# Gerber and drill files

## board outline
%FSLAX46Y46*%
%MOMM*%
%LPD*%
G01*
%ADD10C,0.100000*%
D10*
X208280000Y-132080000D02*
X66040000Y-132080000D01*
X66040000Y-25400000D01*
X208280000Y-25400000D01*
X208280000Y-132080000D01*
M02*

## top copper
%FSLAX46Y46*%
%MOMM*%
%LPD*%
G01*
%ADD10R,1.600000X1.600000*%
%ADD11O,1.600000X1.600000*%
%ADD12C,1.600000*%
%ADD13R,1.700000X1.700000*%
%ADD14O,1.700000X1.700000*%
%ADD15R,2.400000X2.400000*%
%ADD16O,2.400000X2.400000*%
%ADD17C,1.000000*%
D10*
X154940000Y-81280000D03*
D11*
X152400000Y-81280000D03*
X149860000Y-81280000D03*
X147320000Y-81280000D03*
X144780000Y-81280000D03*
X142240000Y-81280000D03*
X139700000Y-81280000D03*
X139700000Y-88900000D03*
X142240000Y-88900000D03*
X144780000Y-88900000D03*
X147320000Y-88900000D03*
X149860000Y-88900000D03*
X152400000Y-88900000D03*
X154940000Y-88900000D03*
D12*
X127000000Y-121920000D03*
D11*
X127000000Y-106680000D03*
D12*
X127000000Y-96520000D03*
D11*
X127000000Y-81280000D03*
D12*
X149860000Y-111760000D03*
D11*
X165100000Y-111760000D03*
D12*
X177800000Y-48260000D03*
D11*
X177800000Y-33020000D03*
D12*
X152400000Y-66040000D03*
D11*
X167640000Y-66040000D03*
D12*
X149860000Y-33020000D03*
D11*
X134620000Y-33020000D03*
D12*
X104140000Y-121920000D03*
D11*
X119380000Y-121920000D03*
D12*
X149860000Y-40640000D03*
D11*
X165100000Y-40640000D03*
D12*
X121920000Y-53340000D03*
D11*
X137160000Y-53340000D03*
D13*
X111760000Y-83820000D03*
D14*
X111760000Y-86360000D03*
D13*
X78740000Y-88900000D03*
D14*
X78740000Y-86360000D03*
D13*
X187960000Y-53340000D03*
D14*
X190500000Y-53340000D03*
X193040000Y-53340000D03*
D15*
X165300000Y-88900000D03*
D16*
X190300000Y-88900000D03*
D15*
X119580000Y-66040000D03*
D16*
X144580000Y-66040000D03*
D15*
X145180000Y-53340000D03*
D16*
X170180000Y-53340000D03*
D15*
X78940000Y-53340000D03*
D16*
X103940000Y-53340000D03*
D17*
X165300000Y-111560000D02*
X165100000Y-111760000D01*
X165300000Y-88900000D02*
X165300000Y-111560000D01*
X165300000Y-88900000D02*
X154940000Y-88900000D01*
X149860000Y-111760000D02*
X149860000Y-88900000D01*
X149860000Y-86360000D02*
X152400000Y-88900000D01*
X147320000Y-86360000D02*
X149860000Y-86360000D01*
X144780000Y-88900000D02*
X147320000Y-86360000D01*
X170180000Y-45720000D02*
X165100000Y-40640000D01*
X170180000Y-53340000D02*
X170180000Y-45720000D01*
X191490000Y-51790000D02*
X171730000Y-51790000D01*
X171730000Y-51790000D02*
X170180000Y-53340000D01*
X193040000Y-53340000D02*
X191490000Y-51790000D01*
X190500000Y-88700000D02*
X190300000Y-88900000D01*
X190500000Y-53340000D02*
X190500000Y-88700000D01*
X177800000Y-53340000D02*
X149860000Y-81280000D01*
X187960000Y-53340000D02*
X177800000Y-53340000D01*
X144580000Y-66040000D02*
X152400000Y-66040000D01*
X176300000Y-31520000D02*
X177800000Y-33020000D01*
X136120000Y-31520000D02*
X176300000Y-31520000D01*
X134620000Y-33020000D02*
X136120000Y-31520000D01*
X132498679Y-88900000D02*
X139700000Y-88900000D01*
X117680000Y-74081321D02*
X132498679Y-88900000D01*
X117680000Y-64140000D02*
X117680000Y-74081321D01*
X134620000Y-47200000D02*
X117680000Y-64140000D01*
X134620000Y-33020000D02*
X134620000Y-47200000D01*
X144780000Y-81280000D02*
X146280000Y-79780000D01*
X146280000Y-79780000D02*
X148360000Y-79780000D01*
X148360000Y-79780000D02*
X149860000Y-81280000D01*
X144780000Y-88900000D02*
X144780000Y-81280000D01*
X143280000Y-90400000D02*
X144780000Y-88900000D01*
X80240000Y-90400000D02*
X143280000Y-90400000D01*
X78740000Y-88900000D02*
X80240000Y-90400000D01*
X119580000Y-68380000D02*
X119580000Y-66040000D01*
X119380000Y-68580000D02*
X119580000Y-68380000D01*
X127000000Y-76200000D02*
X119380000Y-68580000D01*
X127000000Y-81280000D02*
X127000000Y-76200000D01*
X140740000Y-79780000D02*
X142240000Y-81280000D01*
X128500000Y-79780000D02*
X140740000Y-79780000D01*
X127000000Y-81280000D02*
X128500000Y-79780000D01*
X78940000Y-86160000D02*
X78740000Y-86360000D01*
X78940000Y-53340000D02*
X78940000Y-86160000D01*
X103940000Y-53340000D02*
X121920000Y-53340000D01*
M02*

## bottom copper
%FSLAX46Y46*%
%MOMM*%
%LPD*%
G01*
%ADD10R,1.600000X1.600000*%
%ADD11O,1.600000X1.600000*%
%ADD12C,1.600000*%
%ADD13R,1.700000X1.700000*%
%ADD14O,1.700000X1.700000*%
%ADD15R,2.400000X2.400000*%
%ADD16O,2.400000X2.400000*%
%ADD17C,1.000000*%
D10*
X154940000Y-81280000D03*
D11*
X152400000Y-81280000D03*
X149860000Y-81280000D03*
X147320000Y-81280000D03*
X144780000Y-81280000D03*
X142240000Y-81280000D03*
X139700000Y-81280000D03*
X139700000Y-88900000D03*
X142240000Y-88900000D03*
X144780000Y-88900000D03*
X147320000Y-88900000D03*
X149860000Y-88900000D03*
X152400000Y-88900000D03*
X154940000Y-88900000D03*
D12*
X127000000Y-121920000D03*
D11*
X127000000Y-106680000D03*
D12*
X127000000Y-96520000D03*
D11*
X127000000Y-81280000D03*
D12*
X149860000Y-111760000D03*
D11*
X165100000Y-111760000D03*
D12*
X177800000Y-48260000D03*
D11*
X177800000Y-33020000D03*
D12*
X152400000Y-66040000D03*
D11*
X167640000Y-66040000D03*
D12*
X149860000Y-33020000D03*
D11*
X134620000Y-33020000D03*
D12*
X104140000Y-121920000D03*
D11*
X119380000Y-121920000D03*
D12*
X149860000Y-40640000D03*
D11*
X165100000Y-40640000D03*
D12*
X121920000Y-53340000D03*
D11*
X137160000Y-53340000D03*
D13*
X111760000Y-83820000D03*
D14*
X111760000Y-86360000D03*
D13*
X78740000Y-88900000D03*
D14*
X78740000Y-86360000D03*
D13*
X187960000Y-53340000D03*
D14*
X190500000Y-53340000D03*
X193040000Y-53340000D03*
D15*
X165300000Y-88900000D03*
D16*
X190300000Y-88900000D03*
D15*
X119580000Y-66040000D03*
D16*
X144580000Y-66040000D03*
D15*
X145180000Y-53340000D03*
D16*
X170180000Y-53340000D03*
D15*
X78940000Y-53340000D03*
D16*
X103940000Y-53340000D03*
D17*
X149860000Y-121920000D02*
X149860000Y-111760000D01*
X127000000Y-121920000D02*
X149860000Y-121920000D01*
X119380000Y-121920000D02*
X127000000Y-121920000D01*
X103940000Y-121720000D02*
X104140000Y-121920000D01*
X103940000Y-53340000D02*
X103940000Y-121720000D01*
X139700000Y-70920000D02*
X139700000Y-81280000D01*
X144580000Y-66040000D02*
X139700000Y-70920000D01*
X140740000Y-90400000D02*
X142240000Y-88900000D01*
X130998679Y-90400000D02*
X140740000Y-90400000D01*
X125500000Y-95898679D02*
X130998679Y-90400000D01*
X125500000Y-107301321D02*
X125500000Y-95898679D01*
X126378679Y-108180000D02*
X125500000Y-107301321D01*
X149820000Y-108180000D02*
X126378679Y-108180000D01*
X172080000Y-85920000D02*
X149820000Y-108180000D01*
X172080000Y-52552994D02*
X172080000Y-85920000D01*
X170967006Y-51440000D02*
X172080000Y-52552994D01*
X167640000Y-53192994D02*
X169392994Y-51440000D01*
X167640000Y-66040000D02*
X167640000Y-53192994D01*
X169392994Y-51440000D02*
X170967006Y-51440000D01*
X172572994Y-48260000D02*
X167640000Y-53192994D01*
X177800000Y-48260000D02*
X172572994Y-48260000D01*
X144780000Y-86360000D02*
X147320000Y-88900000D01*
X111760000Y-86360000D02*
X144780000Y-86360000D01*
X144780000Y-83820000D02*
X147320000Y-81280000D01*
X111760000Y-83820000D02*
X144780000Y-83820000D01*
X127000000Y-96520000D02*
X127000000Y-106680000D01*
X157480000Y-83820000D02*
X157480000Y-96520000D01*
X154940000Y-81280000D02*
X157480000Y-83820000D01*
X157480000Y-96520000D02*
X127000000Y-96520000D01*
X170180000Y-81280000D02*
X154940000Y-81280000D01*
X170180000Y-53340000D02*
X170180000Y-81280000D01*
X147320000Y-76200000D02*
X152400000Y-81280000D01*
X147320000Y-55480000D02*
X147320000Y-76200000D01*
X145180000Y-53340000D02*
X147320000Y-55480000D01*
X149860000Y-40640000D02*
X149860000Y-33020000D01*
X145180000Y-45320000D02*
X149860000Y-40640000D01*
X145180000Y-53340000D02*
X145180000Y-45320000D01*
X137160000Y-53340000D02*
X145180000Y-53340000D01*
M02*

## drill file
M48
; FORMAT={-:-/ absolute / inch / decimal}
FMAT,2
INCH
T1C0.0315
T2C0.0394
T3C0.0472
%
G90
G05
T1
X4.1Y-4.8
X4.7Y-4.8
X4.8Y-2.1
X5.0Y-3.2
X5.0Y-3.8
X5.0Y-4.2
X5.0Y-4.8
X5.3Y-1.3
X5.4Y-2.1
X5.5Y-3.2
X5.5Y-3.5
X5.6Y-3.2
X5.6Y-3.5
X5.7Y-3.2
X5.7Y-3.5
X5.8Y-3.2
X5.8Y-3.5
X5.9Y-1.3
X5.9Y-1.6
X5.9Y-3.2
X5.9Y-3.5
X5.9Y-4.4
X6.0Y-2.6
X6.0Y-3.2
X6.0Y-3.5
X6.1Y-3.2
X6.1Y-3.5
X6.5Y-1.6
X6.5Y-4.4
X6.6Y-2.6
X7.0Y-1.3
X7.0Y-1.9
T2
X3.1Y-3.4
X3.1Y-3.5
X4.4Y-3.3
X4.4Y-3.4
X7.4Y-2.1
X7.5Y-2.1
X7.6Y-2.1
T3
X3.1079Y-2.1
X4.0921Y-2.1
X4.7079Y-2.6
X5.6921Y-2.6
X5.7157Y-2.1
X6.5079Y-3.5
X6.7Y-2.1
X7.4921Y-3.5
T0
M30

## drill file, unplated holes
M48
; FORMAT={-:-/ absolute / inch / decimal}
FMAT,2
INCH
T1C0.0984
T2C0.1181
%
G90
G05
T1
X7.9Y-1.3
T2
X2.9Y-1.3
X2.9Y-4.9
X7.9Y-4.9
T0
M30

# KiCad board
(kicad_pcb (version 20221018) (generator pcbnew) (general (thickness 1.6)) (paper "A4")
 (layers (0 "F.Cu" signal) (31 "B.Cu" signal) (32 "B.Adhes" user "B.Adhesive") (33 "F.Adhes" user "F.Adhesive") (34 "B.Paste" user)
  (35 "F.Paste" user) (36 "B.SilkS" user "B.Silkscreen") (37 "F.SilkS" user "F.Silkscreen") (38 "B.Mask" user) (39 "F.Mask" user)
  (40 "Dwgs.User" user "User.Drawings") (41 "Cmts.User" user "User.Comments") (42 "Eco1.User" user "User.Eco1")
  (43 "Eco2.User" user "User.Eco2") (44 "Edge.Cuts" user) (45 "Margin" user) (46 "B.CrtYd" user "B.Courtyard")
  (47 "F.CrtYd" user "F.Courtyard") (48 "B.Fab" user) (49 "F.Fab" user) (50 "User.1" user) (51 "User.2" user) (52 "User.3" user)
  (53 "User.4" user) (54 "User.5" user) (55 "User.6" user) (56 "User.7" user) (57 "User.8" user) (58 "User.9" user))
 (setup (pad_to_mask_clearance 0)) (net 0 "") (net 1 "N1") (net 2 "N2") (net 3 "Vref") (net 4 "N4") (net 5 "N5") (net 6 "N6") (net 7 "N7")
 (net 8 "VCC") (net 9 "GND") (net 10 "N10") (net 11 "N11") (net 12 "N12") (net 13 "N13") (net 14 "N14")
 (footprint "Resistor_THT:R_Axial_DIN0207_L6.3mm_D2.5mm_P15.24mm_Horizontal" (layer "F.Cu") (at 152.4 66.04)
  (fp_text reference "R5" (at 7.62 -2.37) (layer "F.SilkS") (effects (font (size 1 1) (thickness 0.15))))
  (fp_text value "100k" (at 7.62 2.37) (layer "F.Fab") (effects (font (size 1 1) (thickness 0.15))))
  (pad "1" thru_hole circle (at 0 0) (size 1.6 1.6) (drill 0.8) (layers "*.Cu" "*.Mask") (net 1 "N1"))
  (pad "2" thru_hole oval (at 15.24 0) (size 1.6 1.6) (drill 0.8) (layers "*.Cu" "*.Mask") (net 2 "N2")))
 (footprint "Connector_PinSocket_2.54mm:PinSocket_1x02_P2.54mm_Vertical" (layer "F.Cu") (at 78.74 88.9 180)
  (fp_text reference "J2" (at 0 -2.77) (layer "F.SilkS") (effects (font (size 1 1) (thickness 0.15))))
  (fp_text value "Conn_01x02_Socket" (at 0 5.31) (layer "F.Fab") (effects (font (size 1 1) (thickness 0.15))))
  (pad "1" thru_hole rect (at 0 0 180) (size 1.7 1.7) (drill 1) (layers "*.Cu" "*.Mask") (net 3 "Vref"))
  (pad "2" thru_hole oval (at 0 2.54 180) (size 1.7 1.7) (drill 1) (layers "*.Cu" "*.Mask") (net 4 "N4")))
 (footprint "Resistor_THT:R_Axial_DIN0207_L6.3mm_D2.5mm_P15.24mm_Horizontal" (layer "F.Cu") (at 121.92 53.34)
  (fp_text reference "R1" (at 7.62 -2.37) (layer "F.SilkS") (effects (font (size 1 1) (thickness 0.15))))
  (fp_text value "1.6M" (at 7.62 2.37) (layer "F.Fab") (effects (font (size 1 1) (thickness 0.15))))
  (pad "1" thru_hole circle (at 0 0) (size 1.6 1.6) (drill 0.8) (layers "*.Cu" "*.Mask") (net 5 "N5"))
  (pad "2" thru_hole oval (at 15.24 0) (size 1.6 1.6) (drill 0.8) (layers "*.Cu" "*.Mask") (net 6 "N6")))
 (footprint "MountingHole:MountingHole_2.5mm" (layer "F.Cu") (at 200.66 33.02)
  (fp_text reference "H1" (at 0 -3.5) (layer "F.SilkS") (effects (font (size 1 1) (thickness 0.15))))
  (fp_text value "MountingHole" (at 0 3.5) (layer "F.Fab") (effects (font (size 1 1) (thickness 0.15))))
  (pad "" np_thru_hole circle (at 0 0) (size 2.5 2.5) (drill 2.5) (layers "*.Cu" "*.Mask")))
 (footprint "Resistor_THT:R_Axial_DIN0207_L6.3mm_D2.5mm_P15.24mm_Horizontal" (layer "F.Cu") (at 149.86 40.64)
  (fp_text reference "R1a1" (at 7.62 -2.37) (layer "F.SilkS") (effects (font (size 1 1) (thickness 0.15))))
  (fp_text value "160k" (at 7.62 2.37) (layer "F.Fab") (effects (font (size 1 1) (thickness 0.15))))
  (pad "1" thru_hole circle (at 0 0) (size 1.6 1.6) (drill 0.8) (layers "*.Cu" "*.Mask") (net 6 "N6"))
  (pad "2" thru_hole oval (at 15.24 0) (size 1.6 1.6) (drill 0.8) (layers "*.Cu" "*.Mask") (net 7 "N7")))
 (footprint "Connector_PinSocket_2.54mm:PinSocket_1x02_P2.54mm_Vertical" (layer "F.Cu") (at 111.76 83.82)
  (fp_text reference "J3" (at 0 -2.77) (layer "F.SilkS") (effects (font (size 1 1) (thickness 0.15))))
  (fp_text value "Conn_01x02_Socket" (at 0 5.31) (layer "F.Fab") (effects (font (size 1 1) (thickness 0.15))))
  (pad "1" thru_hole rect (at 0 0) (size 1.7 1.7) (drill 1) (layers "*.Cu" "*.Mask") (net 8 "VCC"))
  (pad "2" thru_hole oval (at 0 2.54) (size 1.7 1.7) (drill 1) (layers "*.Cu" "*.Mask") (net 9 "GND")))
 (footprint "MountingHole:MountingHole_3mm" (layer "F.Cu") (at 200.66 124.46)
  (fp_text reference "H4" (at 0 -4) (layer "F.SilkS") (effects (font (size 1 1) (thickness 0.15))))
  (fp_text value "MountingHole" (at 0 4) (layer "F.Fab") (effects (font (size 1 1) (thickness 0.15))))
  (pad "" np_thru_hole circle (at 0 0) (size 3 3) (drill 3) (layers "*.Cu" "*.Mask")))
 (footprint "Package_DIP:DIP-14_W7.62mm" (layer "F.Cu") (at 154.94 81.28 -90)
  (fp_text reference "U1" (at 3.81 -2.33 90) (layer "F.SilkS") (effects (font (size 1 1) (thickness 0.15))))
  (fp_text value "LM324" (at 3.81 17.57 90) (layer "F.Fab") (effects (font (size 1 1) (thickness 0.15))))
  (pad "1" thru_hole rect (at 0 0 270) (size 1.6 1.6) (drill 0.8) (layers "*.Cu" "*.Mask") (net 7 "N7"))
  (pad "2" thru_hole oval (at 0 2.54 270) (size 1.6 1.6) (drill 0.8) (layers "*.Cu" "*.Mask") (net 6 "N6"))
  (pad "3" thru_hole oval (at 0 5.08 270) (size 1.6 1.6) (drill 0.8) (layers "*.Cu" "*.Mask") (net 3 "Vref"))
  (pad "4" thru_hole oval (at 0 7.62 270) (size 1.6 1.6) (drill 0.8) (layers "*.Cu" "*.Mask") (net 8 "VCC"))
  (pad "5" thru_hole oval (at 0 10.16 270) (size 1.6 1.6) (drill 0.8) (layers "*.Cu" "*.Mask") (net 3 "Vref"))
  (pad "6" thru_hole oval (at 0 12.7 270) (size 1.6 1.6) (drill 0.8) (layers "*.Cu" "*.Mask") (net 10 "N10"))
  (pad "7" thru_hole oval (at 0 15.24 270) (size 1.6 1.6) (drill 0.8) (layers "*.Cu" "*.Mask") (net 1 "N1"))
  (pad "8" thru_hole oval (at 7.62 15.24 270) (size 1.6 1.6) (drill 0.8) (layers "*.Cu" "*.Mask") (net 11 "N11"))
  (pad "9" thru_hole oval (at 7.62 12.7 270) (size 1.6 1.6) (drill 0.8) (layers "*.Cu" "*.Mask") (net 2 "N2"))
  (pad "10" thru_hole oval (at 7.62 10.16 270) (size 1.6 1.6) (drill 0.8) (layers "*.Cu" "*.Mask") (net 3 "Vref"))
  (pad "11" thru_hole oval (at 7.62 7.62 270) (size 1.6 1.6) (drill 0.8) (layers "*.Cu" "*.Mask") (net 9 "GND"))
  (pad "12" thru_hole oval (at 7.62 5.08 270) (size 1.6 1.6) (drill 0.8) (layers "*.Cu" "*.Mask") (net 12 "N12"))
  (pad "13" thru_hole oval (at 7.62 2.54 270) (size 1.6 1.6) (drill 0.8) (layers "*.Cu" "*.Mask") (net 3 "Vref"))
  (pad "14" thru_hole oval (at 7.62 0 270) (size 1.6 1.6) (drill 0.8) (layers "*.Cu" "*.Mask") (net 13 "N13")))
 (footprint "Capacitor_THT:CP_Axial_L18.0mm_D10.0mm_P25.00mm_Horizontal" (layer "F.Cu") (at 165.3 88.9)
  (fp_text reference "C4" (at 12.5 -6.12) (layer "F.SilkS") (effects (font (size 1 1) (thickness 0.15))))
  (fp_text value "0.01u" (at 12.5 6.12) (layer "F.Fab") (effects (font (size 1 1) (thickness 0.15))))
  (pad "1" thru_hole rect (at 0 0) (size 2.4 2.4) (drill 1.2) (layers "*.Cu" "*.Mask") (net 13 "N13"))
  (pad "2" thru_hole oval (at 25 0) (size 2.4 2.4) (drill 1.2) (layers "*.Cu" "*.Mask") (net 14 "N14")))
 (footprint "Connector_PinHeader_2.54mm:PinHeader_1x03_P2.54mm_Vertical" (layer "F.Cu") (at 187.96 53.34 90)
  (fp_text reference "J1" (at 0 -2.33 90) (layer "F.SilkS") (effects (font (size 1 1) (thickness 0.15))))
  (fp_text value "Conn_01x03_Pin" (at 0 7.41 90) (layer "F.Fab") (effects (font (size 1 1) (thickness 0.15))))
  (pad "1" thru_hole rect (at 0 0 90) (size 1.7 1.7) (drill 1) (layers "*.Cu" "*.Mask") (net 3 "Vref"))
  (pad "2" thru_hole oval (at 0 2.54 90) (size 1.7 1.7) (drill 1) (layers "*.Cu" "*.Mask") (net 14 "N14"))
  (pad "3" thru_hole oval (at 0 5.08 90) (size 1.7 1.7) (drill 1) (layers "*.Cu" "*.Mask") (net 7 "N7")))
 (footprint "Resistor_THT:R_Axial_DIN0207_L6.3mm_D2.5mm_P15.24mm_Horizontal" (layer "F.Cu") (at 104.14 121.92)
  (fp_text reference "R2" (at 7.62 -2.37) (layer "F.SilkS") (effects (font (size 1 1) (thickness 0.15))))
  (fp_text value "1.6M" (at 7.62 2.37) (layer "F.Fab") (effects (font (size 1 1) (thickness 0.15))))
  (pad "1" thru_hole circle (at 0 0) (size 1.6 1.6) (drill 0.8) (layers "*.Cu" "*.Mask") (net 5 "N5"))
  (pad "2" thru_hole oval (at 15.24 0) (size 1.6 1.6) (drill 0.8) (layers "*.Cu" "*.Mask") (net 12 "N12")))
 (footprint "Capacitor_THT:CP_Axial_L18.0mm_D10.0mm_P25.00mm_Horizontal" (layer "F.Cu") (at 78.94 53.34)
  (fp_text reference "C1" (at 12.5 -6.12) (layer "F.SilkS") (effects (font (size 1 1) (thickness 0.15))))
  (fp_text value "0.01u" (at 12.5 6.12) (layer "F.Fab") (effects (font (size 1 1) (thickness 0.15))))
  (pad "1" thru_hole rect (at 0 0) (size 2.4 2.4) (drill 1.2) (layers "*.Cu" "*.Mask") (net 4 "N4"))
  (pad "2" thru_hole oval (at 25 0) (size 2.4 2.4) (drill 1.2) (layers "*.Cu" "*.Mask") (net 5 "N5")))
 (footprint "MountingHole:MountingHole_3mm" (layer "F.Cu") (at 73.66 124.46)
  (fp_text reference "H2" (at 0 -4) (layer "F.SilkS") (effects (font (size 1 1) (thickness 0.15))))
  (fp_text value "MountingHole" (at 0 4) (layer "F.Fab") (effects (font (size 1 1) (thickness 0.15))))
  (pad "" np_thru_hole circle (at 0 0) (size 3 3) (drill 3) (layers "*.Cu" "*.Mask")))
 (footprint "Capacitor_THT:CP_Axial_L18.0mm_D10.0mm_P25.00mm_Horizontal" (layer "F.Cu") (at 145.18 53.34)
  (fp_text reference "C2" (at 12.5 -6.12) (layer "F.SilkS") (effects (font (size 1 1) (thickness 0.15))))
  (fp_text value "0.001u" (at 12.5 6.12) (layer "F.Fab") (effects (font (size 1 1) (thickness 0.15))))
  (pad "1" thru_hole rect (at 0 0) (size 2.4 2.4) (drill 1.2) (layers "*.Cu" "*.Mask") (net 6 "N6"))
  (pad "2" thru_hole oval (at 25 0) (size 2.4 2.4) (drill 1.2) (layers "*.Cu" "*.Mask") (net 7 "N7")))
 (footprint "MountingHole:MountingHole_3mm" (layer "F.Cu") (at 73.66 33.02)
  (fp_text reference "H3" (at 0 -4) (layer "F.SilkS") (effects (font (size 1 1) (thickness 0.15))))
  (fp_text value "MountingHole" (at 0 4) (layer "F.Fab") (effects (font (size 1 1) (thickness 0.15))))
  (pad "" np_thru_hole circle (at 0 0) (size 3 3) (drill 3) (layers "*.Cu" "*.Mask")))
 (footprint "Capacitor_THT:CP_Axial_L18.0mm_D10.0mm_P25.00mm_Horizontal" (layer "F.Cu") (at 119.58 66.04)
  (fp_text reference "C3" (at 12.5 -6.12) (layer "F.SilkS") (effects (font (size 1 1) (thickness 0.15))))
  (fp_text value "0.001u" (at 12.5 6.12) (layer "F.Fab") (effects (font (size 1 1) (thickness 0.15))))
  (pad "1" thru_hole rect (at 0 0) (size 2.4 2.4) (drill 1.2) (layers "*.Cu" "*.Mask") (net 10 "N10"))
  (pad "2" thru_hole oval (at 25 0) (size 2.4 2.4) (drill 1.2) (layers "*.Cu" "*.Mask") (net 1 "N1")))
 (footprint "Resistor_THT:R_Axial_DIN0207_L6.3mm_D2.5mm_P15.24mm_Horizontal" (layer "F.Cu") (at 127 96.52 90)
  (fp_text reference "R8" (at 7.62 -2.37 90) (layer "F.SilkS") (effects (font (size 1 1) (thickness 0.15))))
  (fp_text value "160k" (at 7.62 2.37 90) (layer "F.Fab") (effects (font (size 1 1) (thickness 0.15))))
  (pad "1" thru_hole circle (at 0 0 90) (size 1.6 1.6) (drill 0.8) (layers "*.Cu" "*.Mask") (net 7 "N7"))
  (pad "2" thru_hole oval (at 15.24 0 90) (size 1.6 1.6) (drill 0.8) (layers "*.Cu" "*.Mask") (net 10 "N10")))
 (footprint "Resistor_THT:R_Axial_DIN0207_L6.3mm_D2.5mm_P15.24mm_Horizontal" (layer "F.Cu") (at 149.86 33.02 180)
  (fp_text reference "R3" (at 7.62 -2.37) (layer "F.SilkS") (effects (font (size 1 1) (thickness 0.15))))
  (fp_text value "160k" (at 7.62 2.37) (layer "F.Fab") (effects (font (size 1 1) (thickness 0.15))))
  (pad "1" thru_hole circle (at 0 0 180) (size 1.6 1.6) (drill 0.8) (layers "*.Cu" "*.Mask") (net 6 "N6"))
  (pad "2" thru_hole oval (at 15.24 0 180) (size 1.6 1.6) (drill 0.8) (layers "*.Cu" "*.Mask") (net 11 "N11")))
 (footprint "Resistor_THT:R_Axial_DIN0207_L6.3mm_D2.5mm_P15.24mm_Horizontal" (layer "F.Cu") (at 149.86 111.76)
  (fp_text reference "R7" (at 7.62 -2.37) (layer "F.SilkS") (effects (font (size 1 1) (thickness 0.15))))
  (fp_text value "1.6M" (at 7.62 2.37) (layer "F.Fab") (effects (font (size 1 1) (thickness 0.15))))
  (pad "1" thru_hole circle (at 0 0) (size 1.6 1.6) (drill 0.8) (layers "*.Cu" "*.Mask") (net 12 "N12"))
  (pad "2" thru_hole oval (at 15.24 0) (size 1.6 1.6) (drill 0.8) (layers "*.Cu" "*.Mask") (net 13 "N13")))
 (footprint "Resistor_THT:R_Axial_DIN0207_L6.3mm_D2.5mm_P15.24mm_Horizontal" (layer "F.Cu") (at 177.8 48.26 90)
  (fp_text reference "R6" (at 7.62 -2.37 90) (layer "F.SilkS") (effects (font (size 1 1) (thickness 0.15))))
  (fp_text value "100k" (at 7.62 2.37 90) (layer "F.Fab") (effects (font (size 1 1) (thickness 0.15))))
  (pad "1" thru_hole circle (at 0 0 90) (size 1.6 1.6) (drill 0.8) (layers "*.Cu" "*.Mask") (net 2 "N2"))
  (pad "2" thru_hole oval (at 15.24 0 90) (size 1.6 1.6) (drill 0.8) (layers "*.Cu" "*.Mask") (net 11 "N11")))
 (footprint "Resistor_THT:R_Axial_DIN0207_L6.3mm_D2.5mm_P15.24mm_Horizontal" (layer "F.Cu") (at 127 121.92 90)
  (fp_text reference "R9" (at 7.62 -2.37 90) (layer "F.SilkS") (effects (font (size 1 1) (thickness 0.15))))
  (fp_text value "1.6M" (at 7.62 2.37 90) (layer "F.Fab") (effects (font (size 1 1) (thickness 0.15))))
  (pad "1" thru_hole circle (at 0 0 90) (size 1.6 1.6) (drill 0.8) (layers "*.Cu" "*.Mask") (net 12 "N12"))
  (pad "2" thru_hole oval (at 15.24 0 90) (size 1.6 1.6) (drill 0.8) (layers "*.Cu" "*.Mask") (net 7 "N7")))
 (gr_poly
  (pts (xy 66.04 25.4) (xy 208.28 25.4) (xy 208.28 132.08) (xy 66.04 132.08)) (stroke (width 0.1) (type solid)) (fill none)
  (layer "Edge.Cuts"))
 (segment (start 78.94 86.16) (end 78.74 86.36) (width 1) (layer "F.Cu") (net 4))
 (segment (start 78.94 53.34) (end 78.94 86.16) (width 1) (layer "F.Cu") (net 4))
 (segment (start 103.94 53.34) (end 121.92 53.34) (width 1) (layer "F.Cu") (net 5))
 (segment (start 103.94 53.34) (end 103.94 121.72) (width 1) (layer "B.Cu") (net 5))
 (segment (start 103.94 121.72) (end 104.14 121.92) (width 1) (layer "B.Cu") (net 5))
 (segment (start 147.32 55.48) (end 147.32 76.2) (width 1) (layer "B.Cu") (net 6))
 (segment (start 145.18 53.34) (end 147.32 55.48) (width 1) (layer "B.Cu") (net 6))
 (segment (start 149.86 40.64) (end 149.86 33.02) (width 1) (layer "B.Cu") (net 6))
 (segment (start 137.16 53.34) (end 145.18 53.34) (width 1) (layer "B.Cu") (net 6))
 (segment (start 145.18 45.32) (end 149.86 40.64) (width 1) (layer "B.Cu") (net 6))
 (segment (start 147.32 76.2) (end 152.4 81.28) (width 1) (layer "B.Cu") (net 6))
 (segment (start 145.18 53.34) (end 145.18 45.32) (width 1) (layer "B.Cu") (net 6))
 (segment (start 191.49 51.79) (end 171.73 51.79) (width 1) (layer "F.Cu") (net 7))
 (segment (start 170.18 53.34) (end 170.18 45.72) (width 1) (layer "F.Cu") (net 7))
 (segment (start 171.73 51.79) (end 170.18 53.34) (width 1) (layer "F.Cu") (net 7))
 (segment (start 193.04 53.34) (end 191.49 51.79) (width 1) (layer "F.Cu") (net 7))
 (segment (start 170.18 45.72) (end 165.1 40.64) (width 1) (layer "F.Cu") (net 7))
 (segment (start 154.94 81.28) (end 157.48 83.82) (width 1) (layer "B.Cu") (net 7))
 (segment (start 127 96.52) (end 127 106.68) (width 1) (layer "B.Cu") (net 7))
 (segment (start 157.48 96.52) (end 127 96.52) (width 1) (layer "B.Cu") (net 7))
 (segment (start 170.18 53.34) (end 170.18 81.28) (width 1) (layer "B.Cu") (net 7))
 (segment (start 157.48 83.82) (end 157.48 96.52) (width 1) (layer "B.Cu") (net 7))
 (segment (start 170.18 81.28) (end 154.94 81.28) (width 1) (layer "B.Cu") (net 7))
 (segment (start 128.5 79.78) (end 140.74 79.78) (width 1) (layer "F.Cu") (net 10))
 (segment (start 127 81.28) (end 128.5 79.78) (width 1) (layer "F.Cu") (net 10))
 (segment (start 119.58 68.38) (end 119.58 66.04) (width 1) (layer "F.Cu") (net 10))
 (segment (start 127 81.28) (end 127 76.2) (width 1) (layer "F.Cu") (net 10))
 (segment (start 127 76.2) (end 119.38 68.58) (width 1) (layer "F.Cu") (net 10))
 (segment (start 119.38 68.58) (end 119.58 68.38) (width 1) (layer "F.Cu") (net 10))
 (segment (start 140.74 79.78) (end 142.24 81.28) (width 1) (layer "F.Cu") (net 10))
 (segment (start 144.58 66.04) (end 152.4 66.04) (width 1) (layer "F.Cu") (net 1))
 (segment (start 139.7 70.92) (end 139.7 81.28) (width 1) (layer "B.Cu") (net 1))
 (segment (start 144.58 66.04) (end 139.7 70.92) (width 1) (layer "B.Cu") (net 1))
 (segment (start 165.3 88.9) (end 165.3 111.56) (width 1) (layer "F.Cu") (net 13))
 (segment (start 165.3 111.56) (end 165.1 111.76) (width 1) (layer "F.Cu") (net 13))
 (segment (start 165.3 88.9) (end 154.94 88.9) (width 1) (layer "F.Cu") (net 13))
 (segment (start 190.5 88.7) (end 190.3 88.9) (width 1) (layer "F.Cu") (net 14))
 (segment (start 190.5 53.34) (end 190.5 88.7) (width 1) (layer "F.Cu") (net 14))
 (segment (start 149.86 86.36) (end 152.4 88.9) (width 1) (layer "F.Cu") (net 3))
 (segment (start 146.28 79.78) (end 148.36 79.78) (width 1) (layer "F.Cu") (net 3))
 (segment (start 80.24 90.4) (end 143.28 90.4) (width 1) (layer "F.Cu") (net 3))
 (segment (start 187.96 53.34) (end 177.8 53.34) (width 1) (layer "F.Cu") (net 3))
 (segment (start 143.28 90.4) (end 144.78 88.9) (width 1) (layer "F.Cu") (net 3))
 (segment (start 78.74 88.9) (end 80.24 90.4) (width 1) (layer "F.Cu") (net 3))
 (segment (start 177.8 53.34) (end 149.86 81.28) (width 1) (layer "F.Cu") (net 3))
 (segment (start 144.78 81.28) (end 146.28 79.78) (width 1) (layer "F.Cu") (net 3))
 (segment (start 144.78 88.9) (end 144.78 81.28) (width 1) (layer "F.Cu") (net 3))
 (segment (start 148.36 79.78) (end 149.86 81.28) (width 1) (layer "F.Cu") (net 3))
 (segment (start 144.78 88.9) (end 147.32 86.36) (width 1) (layer "F.Cu") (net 3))
 (segment (start 147.32 86.36) (end 149.86 86.36) (width 1) (layer "F.Cu") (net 3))
 (segment (start 144.78 83.82) (end 147.32 81.28) (width 1) (layer "B.Cu") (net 8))
 (segment (start 111.76 83.82) (end 144.78 83.82) (width 1) (layer "B.Cu") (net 8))
 (segment (start 111.76 86.36) (end 144.78 86.36) (width 1) (layer "B.Cu") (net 9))
 (segment (start 144.78 86.36) (end 147.32 88.9) (width 1) (layer "B.Cu") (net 9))
 (segment (start 149.86 111.76) (end 149.86 88.9) (width 1) (layer "F.Cu") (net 12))
 (segment (start 119.38 121.92) (end 127 121.92) (width 1) (layer "B.Cu") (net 12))
 (segment (start 127 121.92) (end 149.86 121.92) (width 1) (layer "B.Cu") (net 12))
 (segment (start 149.86 121.92) (end 149.86 111.76) (width 1) (layer "B.Cu") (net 12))
 (segment (start 117.68 74.081321) (end 132.498679 88.9) (width 1) (layer "F.Cu") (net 11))
 (segment (start 134.62 47.2) (end 117.68 64.14) (width 1) (layer "F.Cu") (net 11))
 (segment (start 117.68 64.14) (end 117.68 74.081321) (width 1) (layer "F.Cu") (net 11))
 (segment (start 132.498679 88.9) (end 139.7 88.9) (width 1) (layer "F.Cu") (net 11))
 (segment (start 134.62 33.02) (end 136.12 31.52) (width 1) (layer "F.Cu") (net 11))
 (segment (start 136.12 31.52) (end 176.3 31.52) (width 1) (layer "F.Cu") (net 11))
 (segment (start 176.3 31.52) (end 177.8 33.02) (width 1) (layer "F.Cu") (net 11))
 (segment (start 134.62 33.02) (end 134.62 47.2) (width 1) (layer "F.Cu") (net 11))
 (segment (start 125.5 107.301321) (end 125.5 95.898679) (width 1) (layer "B.Cu") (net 2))
 (segment (start 167.64 66.04) (end 167.64 53.192994) (width 1) (layer "B.Cu") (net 2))
 (segment (start 170.967006 51.44) (end 172.08 52.552994) (width 1) (layer "B.Cu") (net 2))
 (segment (start 169.392994 51.44) (end 170.967006 51.44) (width 1) (layer "B.Cu") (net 2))
 (segment (start 177.8 48.26) (end 172.572994 48.26) (width 1) (layer "B.Cu") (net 2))
 (segment (start 125.5 95.898679) (end 130.998679 90.4) (width 1) (layer "B.Cu") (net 2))
 (segment (start 172.08 52.552994) (end 172.08 85.92) (width 1) (layer "B.Cu") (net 2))
 (segment (start 130.998679 90.4) (end 140.74 90.4) (width 1) (layer "B.Cu") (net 2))
 (segment (start 140.74 90.4) (end 142.24 88.9) (width 1) (layer "B.Cu") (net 2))
 (segment (start 126.378679 108.18) (end 125.5 107.301321) (width 1) (layer "B.Cu") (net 2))
 (segment (start 172.08 85.92) (end 149.82 108.18) (width 1) (layer "B.Cu") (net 2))
 (segment (start 172.572994 48.26) (end 167.64 53.192994) (width 1) (layer "B.Cu") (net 2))
 (segment (start 167.64 53.192994) (end 169.392994 51.44) (width 1) (layer "B.Cu") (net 2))
 (segment (start 149.82 108.18) (end 126.378679 108.18) (width 1) (layer "B.Cu") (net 2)))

